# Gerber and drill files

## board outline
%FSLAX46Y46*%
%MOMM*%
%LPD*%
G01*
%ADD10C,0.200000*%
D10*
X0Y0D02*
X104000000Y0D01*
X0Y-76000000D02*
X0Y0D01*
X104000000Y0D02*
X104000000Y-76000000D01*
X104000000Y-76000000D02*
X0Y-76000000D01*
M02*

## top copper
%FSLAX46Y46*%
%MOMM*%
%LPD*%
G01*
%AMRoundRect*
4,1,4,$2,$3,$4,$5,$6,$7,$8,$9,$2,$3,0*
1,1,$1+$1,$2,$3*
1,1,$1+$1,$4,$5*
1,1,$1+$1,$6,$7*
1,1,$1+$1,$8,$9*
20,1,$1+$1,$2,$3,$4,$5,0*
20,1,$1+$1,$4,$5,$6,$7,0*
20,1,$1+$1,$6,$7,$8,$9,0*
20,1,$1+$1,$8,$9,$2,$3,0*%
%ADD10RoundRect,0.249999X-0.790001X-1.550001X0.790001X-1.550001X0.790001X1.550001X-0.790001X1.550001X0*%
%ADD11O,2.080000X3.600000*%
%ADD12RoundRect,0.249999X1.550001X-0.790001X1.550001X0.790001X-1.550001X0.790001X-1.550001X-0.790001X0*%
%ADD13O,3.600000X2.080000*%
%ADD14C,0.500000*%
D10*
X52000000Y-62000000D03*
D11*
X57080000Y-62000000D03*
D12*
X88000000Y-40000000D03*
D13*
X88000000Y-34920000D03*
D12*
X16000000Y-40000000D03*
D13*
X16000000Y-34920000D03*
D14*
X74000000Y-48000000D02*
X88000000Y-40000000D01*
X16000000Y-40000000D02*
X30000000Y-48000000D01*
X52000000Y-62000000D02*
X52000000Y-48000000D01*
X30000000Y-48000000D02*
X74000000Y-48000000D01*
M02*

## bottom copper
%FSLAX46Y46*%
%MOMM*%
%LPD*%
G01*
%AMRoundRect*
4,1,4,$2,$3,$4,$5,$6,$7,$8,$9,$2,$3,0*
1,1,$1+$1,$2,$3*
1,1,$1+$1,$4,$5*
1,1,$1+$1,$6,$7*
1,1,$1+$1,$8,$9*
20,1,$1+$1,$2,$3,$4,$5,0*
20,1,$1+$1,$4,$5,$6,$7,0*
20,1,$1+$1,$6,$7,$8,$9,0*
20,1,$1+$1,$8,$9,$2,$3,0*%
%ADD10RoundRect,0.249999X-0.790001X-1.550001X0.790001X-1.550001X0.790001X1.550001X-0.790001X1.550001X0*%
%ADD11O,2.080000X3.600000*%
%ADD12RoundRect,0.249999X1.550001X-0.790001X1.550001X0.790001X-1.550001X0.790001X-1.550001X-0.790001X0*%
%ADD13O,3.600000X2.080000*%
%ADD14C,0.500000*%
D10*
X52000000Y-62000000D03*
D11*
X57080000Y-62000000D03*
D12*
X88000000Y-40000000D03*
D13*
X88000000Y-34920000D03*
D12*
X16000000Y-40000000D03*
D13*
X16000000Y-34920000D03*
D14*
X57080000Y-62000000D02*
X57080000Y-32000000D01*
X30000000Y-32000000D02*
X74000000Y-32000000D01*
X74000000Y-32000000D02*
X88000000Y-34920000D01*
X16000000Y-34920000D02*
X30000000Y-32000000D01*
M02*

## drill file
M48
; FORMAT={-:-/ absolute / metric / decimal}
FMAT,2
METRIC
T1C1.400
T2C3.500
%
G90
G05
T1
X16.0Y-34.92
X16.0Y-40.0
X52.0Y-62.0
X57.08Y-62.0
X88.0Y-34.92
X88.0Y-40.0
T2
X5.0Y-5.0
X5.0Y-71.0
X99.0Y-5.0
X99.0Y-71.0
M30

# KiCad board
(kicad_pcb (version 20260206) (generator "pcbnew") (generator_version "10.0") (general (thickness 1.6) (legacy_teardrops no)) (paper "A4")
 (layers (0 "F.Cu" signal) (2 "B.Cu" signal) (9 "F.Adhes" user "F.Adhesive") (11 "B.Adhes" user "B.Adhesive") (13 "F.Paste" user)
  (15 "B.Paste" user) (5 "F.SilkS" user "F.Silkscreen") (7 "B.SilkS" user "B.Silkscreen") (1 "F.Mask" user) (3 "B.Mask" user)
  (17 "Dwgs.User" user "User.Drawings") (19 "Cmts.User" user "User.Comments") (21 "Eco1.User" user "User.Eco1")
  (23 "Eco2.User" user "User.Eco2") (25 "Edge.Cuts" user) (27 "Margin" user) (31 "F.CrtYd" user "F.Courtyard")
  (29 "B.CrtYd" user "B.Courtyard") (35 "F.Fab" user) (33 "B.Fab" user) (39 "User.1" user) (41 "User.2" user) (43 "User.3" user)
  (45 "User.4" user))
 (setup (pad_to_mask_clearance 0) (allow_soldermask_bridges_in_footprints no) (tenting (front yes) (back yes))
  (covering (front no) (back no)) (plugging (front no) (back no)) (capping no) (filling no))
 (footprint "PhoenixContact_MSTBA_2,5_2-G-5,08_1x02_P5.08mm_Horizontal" (layer "F.Cu") (at 52 62)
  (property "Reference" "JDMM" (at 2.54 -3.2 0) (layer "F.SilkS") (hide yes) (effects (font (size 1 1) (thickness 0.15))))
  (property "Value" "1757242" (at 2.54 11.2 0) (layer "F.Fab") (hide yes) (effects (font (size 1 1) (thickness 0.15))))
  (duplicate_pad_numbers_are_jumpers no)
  (pad "1" thru_hole roundrect (at 0 0) (size 2.08 3.6) (drill 1.4) (layers "*.Cu" "*.Mask") (remove_unused_layers no)
   (roundrect_rratio 0.120192) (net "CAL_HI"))
  (pad "2" thru_hole oval (at 5.08 0) (size 2.08 3.6) (drill 1.4) (layers "*.Cu" "*.Mask") (remove_unused_layers no) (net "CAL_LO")))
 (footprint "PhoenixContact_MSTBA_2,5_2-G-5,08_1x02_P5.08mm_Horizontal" (layer "F.Cu") (at 88 40 90)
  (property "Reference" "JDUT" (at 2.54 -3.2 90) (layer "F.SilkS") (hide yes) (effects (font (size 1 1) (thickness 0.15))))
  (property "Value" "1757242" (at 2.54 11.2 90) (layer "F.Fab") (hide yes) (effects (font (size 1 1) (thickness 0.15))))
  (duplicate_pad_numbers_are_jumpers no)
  (pad "1" thru_hole roundrect (at 0 0 90) (size 2.08 3.6) (drill 1.4) (layers "*.Cu" "*.Mask") (remove_unused_layers no)
   (roundrect_rratio 0.120192) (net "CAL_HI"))
  (pad "2" thru_hole oval (at 5.08 0 90) (size 2.08 3.6) (drill 1.4) (layers "*.Cu" "*.Mask") (remove_unused_layers no) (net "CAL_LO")))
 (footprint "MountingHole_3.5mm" (layer "F.Cu") (at 5 71)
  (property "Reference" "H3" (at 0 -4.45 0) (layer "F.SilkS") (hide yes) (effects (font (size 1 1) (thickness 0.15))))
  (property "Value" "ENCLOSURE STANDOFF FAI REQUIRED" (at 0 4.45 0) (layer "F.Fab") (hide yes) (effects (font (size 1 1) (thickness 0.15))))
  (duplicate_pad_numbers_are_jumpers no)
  (pad "" np_thru_hole circle (at 0 0) (size 3.5 3.5) (drill 3.5) (layers "*.Cu" "*.Mask")))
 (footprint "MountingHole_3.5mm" (layer "F.Cu") (at 99 71)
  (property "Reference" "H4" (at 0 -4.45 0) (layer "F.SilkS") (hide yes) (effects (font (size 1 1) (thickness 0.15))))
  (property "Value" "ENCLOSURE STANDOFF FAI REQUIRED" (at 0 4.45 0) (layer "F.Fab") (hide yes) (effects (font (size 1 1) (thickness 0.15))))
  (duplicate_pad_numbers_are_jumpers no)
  (pad "" np_thru_hole circle (at 0 0) (size 3.5 3.5) (drill 3.5) (layers "*.Cu" "*.Mask")))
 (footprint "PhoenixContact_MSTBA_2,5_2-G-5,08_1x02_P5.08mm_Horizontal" (layer "F.Cu") (at 16 40 90)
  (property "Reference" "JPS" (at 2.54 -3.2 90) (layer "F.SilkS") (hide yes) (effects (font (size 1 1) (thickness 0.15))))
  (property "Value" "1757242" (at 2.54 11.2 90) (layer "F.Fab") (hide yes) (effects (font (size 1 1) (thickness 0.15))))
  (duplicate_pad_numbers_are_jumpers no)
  (pad "1" thru_hole roundrect (at 0 0 90) (size 2.08 3.6) (drill 1.4) (layers "*.Cu" "*.Mask") (remove_unused_layers no)
   (roundrect_rratio 0.120192) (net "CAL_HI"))
  (pad "2" thru_hole oval (at 5.08 0 90) (size 2.08 3.6) (drill 1.4) (layers "*.Cu" "*.Mask") (remove_unused_layers no) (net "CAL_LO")))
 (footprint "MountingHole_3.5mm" (layer "F.Cu") (at 99 5)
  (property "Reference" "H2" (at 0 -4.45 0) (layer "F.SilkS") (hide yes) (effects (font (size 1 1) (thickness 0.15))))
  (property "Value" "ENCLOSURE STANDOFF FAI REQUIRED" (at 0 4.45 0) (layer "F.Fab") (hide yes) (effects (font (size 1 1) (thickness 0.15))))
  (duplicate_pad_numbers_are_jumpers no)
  (pad "" np_thru_hole circle (at 0 0) (size 3.5 3.5) (drill 3.5) (layers "*.Cu" "*.Mask")))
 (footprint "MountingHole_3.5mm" (layer "F.Cu") (at 5 5)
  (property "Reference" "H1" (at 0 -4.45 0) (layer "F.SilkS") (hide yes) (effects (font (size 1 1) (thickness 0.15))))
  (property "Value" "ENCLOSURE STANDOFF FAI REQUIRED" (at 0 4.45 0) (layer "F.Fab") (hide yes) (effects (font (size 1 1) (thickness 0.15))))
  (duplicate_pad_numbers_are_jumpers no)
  (pad "" np_thru_hole circle (at 0 0) (size 3.5 3.5) (drill 3.5) (layers "*.Cu" "*.Mask")))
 (gr_line (start 0 0) (end 104 0) (stroke (width 0.2) (type default)) (layer "Edge.Cuts"))
 (gr_line (start 0 76) (end 0 0) (stroke (width 0.2) (type default)) (layer "Edge.Cuts"))
 (gr_line (start 104 0) (end 104 76) (stroke (width 0.2) (type default)) (layer "Edge.Cuts"))
 (gr_line (start 104 76) (end 0 76) (stroke (width 0.2) (type default)) (layer "Edge.Cuts"))
 (segment (start 74 48) (end 88 40) (width 0.5) (layer "F.Cu") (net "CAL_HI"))
 (segment (start 16 40) (end 30 48) (width 0.5) (layer "F.Cu") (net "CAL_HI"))
 (segment (start 52 62) (end 52 48) (width 0.5) (layer "F.Cu") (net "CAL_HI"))
 (segment (start 30 48) (end 74 48) (width 0.5) (layer "F.Cu") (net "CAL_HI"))
 (segment (start 57.08 62) (end 57.08 32) (width 0.5) (layer "B.Cu") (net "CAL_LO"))
 (segment (start 30 32) (end 74 32) (width 0.5) (layer "B.Cu") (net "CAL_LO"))
 (segment (start 74 32) (end 88 34.92) (width 0.5) (layer "B.Cu") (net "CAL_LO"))
 (segment (start 16 34.92) (end 30 32) (width 0.5) (layer "B.Cu") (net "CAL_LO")))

